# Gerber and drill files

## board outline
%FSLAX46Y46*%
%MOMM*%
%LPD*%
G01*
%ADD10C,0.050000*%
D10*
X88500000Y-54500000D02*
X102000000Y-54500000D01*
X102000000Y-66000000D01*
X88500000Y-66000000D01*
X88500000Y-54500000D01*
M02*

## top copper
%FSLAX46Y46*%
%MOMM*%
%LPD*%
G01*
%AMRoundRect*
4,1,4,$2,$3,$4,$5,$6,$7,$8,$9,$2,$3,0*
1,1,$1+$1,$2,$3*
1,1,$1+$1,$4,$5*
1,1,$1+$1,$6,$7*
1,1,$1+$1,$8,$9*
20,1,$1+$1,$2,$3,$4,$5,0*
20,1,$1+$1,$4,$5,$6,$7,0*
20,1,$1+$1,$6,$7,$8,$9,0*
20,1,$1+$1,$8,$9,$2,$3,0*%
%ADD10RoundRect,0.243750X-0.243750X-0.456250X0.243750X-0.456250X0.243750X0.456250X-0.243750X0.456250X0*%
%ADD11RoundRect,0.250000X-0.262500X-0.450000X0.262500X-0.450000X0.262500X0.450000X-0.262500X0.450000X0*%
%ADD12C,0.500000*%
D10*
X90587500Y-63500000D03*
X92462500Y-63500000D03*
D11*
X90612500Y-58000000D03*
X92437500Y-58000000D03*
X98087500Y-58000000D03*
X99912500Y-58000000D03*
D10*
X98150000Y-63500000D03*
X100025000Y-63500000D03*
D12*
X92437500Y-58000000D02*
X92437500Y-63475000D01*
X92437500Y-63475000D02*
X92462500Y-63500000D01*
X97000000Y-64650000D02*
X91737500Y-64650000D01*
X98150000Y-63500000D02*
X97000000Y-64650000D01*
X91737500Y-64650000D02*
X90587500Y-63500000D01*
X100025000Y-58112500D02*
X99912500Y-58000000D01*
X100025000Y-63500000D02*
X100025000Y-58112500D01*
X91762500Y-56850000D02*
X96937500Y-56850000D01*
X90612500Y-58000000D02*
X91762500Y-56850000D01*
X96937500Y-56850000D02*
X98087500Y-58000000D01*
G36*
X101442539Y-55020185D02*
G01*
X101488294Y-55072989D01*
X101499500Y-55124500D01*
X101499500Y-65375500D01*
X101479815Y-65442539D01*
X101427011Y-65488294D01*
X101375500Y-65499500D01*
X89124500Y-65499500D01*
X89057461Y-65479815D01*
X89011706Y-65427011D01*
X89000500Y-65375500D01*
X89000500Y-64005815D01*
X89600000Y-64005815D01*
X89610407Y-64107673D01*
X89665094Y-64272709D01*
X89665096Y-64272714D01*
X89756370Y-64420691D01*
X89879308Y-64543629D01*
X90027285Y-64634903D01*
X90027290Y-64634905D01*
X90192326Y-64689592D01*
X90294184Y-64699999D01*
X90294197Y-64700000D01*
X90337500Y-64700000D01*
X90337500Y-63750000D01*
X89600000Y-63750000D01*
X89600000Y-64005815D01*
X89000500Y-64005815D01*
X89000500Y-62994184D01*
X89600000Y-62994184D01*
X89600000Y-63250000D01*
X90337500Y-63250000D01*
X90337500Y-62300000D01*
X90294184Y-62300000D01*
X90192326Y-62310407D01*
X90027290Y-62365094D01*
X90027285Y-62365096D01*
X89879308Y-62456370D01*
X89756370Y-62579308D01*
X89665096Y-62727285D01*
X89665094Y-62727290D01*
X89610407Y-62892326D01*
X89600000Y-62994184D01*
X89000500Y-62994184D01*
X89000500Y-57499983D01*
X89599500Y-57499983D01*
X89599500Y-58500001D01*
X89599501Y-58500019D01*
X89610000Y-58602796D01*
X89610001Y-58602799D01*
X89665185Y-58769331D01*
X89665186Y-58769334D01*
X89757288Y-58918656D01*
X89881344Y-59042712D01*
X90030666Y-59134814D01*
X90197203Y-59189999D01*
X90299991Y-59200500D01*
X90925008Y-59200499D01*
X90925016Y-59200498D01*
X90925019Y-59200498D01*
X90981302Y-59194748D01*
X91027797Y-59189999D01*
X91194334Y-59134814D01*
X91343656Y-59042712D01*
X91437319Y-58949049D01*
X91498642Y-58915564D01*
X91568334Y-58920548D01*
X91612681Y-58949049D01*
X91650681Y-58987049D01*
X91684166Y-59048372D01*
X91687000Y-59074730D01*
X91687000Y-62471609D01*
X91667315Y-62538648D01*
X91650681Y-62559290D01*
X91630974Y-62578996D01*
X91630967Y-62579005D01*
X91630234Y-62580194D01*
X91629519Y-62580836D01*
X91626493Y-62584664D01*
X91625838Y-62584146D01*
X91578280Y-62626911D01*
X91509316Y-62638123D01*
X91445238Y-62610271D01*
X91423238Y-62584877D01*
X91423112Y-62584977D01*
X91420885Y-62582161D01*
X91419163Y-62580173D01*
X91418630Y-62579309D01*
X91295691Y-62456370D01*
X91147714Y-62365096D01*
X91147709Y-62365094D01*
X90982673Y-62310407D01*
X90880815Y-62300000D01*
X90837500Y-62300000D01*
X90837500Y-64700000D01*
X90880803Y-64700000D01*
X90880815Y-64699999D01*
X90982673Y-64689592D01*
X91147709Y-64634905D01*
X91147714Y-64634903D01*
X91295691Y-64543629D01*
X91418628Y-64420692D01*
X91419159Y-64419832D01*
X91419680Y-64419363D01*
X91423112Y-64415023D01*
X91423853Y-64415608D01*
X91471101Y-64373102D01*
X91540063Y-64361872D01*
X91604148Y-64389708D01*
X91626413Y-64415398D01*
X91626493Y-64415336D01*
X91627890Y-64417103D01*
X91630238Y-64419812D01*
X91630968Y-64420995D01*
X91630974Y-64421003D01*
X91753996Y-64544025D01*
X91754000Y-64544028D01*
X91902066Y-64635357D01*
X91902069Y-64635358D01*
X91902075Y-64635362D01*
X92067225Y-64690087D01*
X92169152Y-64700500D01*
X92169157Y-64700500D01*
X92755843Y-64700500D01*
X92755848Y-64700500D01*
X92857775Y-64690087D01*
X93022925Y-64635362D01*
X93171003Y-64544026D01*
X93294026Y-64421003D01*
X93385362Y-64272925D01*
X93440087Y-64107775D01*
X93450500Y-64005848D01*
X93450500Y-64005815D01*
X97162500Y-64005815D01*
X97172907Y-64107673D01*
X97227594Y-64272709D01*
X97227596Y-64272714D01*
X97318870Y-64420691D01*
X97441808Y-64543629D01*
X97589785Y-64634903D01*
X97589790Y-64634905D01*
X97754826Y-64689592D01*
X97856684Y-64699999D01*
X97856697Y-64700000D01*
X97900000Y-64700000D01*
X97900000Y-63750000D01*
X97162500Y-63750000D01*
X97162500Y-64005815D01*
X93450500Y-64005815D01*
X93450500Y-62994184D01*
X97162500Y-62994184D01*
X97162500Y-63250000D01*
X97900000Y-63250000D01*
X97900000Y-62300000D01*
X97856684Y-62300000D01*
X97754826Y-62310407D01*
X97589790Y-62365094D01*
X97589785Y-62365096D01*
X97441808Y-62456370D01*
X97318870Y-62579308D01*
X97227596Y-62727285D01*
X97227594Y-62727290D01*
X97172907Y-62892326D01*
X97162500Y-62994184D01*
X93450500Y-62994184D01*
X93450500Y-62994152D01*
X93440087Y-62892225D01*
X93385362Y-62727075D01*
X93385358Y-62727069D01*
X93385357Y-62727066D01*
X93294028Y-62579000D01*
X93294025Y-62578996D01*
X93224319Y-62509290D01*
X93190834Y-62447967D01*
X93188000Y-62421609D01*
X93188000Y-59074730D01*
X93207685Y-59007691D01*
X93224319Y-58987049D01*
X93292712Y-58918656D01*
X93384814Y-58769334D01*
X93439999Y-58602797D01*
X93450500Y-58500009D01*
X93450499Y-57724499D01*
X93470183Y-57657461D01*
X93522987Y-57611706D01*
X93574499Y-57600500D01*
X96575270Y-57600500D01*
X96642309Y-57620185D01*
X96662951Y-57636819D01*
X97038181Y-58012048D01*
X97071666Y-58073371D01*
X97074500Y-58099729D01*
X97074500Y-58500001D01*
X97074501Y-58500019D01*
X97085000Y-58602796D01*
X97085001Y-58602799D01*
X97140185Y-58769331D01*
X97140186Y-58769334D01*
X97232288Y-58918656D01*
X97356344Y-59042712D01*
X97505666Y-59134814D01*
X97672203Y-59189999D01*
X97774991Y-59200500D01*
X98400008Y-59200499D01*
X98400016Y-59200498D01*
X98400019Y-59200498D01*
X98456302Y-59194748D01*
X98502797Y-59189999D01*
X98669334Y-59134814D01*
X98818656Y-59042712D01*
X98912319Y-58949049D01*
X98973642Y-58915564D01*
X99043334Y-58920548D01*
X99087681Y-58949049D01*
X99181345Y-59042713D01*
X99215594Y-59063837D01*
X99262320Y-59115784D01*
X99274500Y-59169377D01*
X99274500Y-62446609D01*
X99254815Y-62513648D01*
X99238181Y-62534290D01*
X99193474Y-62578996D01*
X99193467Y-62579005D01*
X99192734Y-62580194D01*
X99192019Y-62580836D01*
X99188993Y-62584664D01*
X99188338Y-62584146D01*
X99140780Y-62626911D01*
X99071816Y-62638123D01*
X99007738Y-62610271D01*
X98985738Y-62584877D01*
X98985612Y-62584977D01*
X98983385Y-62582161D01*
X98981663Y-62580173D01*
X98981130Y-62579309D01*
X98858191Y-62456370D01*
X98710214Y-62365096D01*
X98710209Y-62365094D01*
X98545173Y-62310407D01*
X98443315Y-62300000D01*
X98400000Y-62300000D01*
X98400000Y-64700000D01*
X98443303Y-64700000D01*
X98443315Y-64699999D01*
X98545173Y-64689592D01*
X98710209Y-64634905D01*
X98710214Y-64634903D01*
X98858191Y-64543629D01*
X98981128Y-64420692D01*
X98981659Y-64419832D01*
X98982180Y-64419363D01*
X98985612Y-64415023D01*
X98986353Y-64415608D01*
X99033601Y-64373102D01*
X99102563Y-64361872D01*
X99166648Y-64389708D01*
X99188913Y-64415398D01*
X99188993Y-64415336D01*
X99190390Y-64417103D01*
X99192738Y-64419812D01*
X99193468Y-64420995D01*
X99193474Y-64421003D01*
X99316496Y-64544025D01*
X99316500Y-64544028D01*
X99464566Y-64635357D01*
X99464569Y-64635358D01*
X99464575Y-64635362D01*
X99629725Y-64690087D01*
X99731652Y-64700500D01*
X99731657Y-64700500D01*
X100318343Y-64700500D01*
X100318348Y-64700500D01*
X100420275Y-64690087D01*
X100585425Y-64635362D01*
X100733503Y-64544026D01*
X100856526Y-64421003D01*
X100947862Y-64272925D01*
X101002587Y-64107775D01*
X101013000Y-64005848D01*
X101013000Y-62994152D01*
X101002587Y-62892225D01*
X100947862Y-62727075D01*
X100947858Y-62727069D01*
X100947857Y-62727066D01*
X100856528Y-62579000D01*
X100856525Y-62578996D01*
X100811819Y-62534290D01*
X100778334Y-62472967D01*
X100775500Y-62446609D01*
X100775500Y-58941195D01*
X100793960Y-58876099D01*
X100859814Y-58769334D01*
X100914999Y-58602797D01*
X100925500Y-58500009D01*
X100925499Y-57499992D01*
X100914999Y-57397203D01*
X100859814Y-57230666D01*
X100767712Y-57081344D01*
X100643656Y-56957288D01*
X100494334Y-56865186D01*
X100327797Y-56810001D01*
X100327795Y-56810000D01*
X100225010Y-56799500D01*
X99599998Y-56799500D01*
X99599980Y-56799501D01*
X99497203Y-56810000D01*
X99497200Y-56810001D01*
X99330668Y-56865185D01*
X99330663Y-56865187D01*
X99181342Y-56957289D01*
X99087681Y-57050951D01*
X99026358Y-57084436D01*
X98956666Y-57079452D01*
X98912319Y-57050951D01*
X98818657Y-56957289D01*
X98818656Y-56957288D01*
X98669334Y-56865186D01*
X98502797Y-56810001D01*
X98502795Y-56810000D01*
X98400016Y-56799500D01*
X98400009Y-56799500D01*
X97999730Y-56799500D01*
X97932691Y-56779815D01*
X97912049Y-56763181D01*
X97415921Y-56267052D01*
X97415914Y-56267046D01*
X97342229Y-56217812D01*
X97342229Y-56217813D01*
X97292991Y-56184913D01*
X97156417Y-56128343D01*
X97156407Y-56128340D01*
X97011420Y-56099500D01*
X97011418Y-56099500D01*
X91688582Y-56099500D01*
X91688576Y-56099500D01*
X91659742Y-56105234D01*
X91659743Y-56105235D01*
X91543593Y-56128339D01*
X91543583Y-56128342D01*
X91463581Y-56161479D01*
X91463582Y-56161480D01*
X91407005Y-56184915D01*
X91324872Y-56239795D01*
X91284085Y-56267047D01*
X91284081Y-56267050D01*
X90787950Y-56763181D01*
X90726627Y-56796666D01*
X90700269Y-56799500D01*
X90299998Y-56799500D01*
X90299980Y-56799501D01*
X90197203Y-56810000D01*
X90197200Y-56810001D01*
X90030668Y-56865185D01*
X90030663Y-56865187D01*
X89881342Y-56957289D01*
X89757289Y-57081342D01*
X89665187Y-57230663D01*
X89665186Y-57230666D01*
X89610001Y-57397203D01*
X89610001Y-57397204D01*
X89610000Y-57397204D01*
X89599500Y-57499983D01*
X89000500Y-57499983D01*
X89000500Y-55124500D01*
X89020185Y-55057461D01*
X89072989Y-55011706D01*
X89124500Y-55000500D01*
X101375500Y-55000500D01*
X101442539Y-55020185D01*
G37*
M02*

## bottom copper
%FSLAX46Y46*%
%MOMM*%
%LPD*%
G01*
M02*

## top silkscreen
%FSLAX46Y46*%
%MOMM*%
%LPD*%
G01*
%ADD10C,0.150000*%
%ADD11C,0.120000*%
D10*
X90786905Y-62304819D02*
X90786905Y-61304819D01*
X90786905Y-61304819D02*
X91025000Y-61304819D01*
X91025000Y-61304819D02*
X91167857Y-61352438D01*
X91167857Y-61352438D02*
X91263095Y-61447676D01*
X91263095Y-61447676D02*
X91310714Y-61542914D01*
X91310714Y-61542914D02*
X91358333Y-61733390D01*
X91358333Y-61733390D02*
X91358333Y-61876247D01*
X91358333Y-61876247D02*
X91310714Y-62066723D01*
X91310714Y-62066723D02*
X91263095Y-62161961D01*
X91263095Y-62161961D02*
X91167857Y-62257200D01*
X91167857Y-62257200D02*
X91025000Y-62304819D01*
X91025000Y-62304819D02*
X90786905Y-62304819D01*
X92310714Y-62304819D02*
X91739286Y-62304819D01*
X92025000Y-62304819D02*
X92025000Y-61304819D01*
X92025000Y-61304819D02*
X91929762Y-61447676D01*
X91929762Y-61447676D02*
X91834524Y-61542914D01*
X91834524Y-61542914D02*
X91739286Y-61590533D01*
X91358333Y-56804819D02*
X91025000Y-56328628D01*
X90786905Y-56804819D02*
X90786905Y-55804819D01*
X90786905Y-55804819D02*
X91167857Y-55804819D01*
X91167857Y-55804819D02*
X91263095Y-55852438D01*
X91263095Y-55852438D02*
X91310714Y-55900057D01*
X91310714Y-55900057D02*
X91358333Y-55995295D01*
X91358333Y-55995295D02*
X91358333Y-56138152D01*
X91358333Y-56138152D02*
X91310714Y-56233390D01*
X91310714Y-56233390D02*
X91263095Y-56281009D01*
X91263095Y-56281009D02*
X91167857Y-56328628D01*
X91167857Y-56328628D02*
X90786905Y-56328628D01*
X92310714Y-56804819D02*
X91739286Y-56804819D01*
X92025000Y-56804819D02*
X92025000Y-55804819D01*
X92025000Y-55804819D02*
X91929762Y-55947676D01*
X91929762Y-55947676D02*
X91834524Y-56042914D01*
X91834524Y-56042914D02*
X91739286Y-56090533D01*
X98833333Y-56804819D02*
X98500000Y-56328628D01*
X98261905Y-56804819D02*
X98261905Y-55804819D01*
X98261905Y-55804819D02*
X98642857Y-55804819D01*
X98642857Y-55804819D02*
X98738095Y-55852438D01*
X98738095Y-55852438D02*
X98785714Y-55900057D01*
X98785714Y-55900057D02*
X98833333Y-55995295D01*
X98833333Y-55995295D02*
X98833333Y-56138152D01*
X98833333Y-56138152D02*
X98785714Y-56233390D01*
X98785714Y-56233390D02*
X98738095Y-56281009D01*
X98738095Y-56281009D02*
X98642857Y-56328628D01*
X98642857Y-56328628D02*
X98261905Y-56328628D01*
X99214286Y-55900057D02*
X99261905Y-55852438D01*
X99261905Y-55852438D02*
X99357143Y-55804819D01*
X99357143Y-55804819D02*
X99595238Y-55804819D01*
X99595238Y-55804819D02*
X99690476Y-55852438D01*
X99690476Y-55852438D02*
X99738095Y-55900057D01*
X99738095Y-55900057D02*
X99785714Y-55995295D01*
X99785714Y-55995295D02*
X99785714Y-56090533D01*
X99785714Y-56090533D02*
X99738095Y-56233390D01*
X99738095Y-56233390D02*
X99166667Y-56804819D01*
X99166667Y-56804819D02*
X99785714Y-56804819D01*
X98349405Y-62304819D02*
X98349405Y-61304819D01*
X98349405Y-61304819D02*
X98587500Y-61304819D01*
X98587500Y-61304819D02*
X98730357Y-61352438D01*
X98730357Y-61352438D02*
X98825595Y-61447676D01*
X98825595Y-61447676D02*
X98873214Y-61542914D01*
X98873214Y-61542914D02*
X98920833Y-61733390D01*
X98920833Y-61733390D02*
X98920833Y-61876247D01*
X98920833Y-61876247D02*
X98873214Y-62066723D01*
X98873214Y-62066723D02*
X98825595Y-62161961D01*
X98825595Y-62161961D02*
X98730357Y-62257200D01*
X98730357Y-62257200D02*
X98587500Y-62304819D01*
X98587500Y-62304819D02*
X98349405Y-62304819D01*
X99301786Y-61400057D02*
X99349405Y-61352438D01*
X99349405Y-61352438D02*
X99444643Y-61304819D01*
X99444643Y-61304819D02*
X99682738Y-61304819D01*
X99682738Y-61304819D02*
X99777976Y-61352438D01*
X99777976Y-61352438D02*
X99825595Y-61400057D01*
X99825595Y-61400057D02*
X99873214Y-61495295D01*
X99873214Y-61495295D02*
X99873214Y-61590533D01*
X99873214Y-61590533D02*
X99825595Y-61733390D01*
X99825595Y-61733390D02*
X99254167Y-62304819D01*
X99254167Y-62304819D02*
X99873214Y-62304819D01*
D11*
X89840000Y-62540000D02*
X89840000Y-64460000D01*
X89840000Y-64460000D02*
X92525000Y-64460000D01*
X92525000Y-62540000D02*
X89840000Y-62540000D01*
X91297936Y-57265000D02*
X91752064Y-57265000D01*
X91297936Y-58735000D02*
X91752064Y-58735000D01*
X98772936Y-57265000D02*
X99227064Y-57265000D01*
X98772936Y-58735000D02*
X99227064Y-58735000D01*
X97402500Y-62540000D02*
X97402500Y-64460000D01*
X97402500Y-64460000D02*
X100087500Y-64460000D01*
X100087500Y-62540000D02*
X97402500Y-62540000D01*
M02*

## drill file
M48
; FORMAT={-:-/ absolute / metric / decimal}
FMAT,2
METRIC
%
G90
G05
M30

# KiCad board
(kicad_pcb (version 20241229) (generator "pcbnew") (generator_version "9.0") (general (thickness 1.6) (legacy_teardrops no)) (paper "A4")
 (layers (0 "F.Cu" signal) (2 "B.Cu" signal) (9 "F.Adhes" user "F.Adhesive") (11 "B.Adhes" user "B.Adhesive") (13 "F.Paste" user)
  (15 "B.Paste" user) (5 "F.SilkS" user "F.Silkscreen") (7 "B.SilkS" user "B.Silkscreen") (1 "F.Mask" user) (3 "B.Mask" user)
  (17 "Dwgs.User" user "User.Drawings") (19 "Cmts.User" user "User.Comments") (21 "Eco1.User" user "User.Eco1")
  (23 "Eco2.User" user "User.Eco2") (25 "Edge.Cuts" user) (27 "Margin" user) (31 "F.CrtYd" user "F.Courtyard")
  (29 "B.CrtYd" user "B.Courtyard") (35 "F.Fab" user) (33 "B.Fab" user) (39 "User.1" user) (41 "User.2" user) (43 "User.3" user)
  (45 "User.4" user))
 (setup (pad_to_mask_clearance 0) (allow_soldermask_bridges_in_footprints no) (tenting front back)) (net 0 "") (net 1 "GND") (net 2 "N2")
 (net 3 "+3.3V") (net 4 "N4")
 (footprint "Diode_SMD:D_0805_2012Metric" (layer "F.Cu") (at 91.525 63.5)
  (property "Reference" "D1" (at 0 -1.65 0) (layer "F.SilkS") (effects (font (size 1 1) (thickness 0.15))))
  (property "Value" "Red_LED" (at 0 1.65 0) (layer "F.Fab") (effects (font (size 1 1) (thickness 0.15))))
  (fp_line (start -1.685 -0.96) (end -1.685 0.96) (stroke (width 0.12) (type solid)) (layer "F.SilkS"))
  (fp_line (start -1.685 0.96) (end 1 0.96) (stroke (width 0.12) (type solid)) (layer "F.SilkS"))
  (fp_line (start 1 -0.96) (end -1.685 -0.96) (stroke (width 0.12) (type solid)) (layer "F.SilkS"))
  (pad "1" smd roundrect (at -0.9375 0) (size 0.975 1.4) (layers "F.Cu" "F.Mask" "F.Paste") (roundrect_rratio 0.25) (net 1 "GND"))
  (pad "2" smd roundrect (at 0.9375 0) (size 0.975 1.4) (layers "F.Cu" "F.Mask" "F.Paste") (roundrect_rratio 0.25) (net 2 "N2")))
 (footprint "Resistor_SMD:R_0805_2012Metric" (layer "F.Cu") (at 91.525 58)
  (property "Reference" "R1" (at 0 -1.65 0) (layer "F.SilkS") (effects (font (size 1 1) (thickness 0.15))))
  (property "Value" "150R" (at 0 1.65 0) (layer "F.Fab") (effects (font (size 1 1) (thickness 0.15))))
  (fp_line (start -0.227064 -0.735) (end 0.227064 -0.735) (stroke (width 0.12) (type solid)) (layer "F.SilkS"))
  (fp_line (start -0.227064 0.735) (end 0.227064 0.735) (stroke (width 0.12) (type solid)) (layer "F.SilkS"))
  (pad "1" smd roundrect (at -0.9125 0) (size 1.025 1.4) (layers "F.Cu" "F.Mask" "F.Paste") (roundrect_rratio 0.243902) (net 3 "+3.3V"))
  (pad "2" smd roundrect (at 0.9125 0) (size 1.025 1.4) (layers "F.Cu" "F.Mask" "F.Paste") (roundrect_rratio 0.243902) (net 2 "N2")))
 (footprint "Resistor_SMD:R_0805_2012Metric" (layer "F.Cu") (at 99 58)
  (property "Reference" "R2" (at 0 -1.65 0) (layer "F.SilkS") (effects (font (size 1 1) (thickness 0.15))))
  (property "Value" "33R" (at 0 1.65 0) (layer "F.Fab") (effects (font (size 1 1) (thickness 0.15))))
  (fp_line (start -0.227064 -0.735) (end 0.227064 -0.735) (stroke (width 0.12) (type solid)) (layer "F.SilkS"))
  (fp_line (start -0.227064 0.735) (end 0.227064 0.735) (stroke (width 0.12) (type solid)) (layer "F.SilkS"))
  (pad "1" smd roundrect (at -0.9125 0) (size 1.025 1.4) (layers "F.Cu" "F.Mask" "F.Paste") (roundrect_rratio 0.243902) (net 3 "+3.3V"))
  (pad "2" smd roundrect (at 0.9125 0) (size 1.025 1.4) (layers "F.Cu" "F.Mask" "F.Paste") (roundrect_rratio 0.243902) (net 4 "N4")))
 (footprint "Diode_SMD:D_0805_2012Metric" (layer "F.Cu") (at 99.0875 63.5)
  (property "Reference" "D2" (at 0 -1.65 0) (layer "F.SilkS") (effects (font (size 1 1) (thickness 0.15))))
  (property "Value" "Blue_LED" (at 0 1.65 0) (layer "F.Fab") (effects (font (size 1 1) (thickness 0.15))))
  (fp_line (start -1.685 -0.96) (end -1.685 0.96) (stroke (width 0.12) (type solid)) (layer "F.SilkS"))
  (fp_line (start -1.685 0.96) (end 1 0.96) (stroke (width 0.12) (type solid)) (layer "F.SilkS"))
  (fp_line (start 1 -0.96) (end -1.685 -0.96) (stroke (width 0.12) (type solid)) (layer "F.SilkS"))
  (pad "1" smd roundrect (at -0.9375 0) (size 0.975 1.4) (layers "F.Cu" "F.Mask" "F.Paste") (roundrect_rratio 0.25) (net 1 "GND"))
  (pad "2" smd roundrect (at 0.9375 0) (size 0.975 1.4) (layers "F.Cu" "F.Mask" "F.Paste") (roundrect_rratio 0.25) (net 4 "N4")))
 (gr_rect (start 88.5 54.5) (end 102 66) (stroke (width 0.05) (type solid)) (fill no) (layer "Edge.Cuts"))
 (segment (start 92.4375 58) (end 92.4375 63.475) (width 0.5) (layer "F.Cu") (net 2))
 (segment (start 92.4375 63.475) (end 92.4625 63.5) (width 0.5) (layer "F.Cu") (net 2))
 (segment (start 97 64.65) (end 91.7375 64.65) (width 0.5) (layer "F.Cu") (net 1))
 (segment (start 98.15 63.5) (end 97 64.65) (width 0.5) (layer "F.Cu") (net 1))
 (segment (start 91.7375 64.65) (end 90.5875 63.5) (width 0.5) (layer "F.Cu") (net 1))
 (segment (start 100.025 58.1125) (end 99.9125 58) (width 0.5) (layer "F.Cu") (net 4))
 (segment (start 100.025 63.5) (end 100.025 58.1125) (width 0.5) (layer "F.Cu") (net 4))
 (segment (start 91.7625 56.85) (end 96.9375 56.85) (width 0.5) (layer "F.Cu") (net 3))
 (segment (start 90.6125 58) (end 91.7625 56.85) (width 0.5) (layer "F.Cu") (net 3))
 (segment (start 96.9375 56.85) (end 98.0875 58) (width 0.5) (layer "F.Cu") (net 3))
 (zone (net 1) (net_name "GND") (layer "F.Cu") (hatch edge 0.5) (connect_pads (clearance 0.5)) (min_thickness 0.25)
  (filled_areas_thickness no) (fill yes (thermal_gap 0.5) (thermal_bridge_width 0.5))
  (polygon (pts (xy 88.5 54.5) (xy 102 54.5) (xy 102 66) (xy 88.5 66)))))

